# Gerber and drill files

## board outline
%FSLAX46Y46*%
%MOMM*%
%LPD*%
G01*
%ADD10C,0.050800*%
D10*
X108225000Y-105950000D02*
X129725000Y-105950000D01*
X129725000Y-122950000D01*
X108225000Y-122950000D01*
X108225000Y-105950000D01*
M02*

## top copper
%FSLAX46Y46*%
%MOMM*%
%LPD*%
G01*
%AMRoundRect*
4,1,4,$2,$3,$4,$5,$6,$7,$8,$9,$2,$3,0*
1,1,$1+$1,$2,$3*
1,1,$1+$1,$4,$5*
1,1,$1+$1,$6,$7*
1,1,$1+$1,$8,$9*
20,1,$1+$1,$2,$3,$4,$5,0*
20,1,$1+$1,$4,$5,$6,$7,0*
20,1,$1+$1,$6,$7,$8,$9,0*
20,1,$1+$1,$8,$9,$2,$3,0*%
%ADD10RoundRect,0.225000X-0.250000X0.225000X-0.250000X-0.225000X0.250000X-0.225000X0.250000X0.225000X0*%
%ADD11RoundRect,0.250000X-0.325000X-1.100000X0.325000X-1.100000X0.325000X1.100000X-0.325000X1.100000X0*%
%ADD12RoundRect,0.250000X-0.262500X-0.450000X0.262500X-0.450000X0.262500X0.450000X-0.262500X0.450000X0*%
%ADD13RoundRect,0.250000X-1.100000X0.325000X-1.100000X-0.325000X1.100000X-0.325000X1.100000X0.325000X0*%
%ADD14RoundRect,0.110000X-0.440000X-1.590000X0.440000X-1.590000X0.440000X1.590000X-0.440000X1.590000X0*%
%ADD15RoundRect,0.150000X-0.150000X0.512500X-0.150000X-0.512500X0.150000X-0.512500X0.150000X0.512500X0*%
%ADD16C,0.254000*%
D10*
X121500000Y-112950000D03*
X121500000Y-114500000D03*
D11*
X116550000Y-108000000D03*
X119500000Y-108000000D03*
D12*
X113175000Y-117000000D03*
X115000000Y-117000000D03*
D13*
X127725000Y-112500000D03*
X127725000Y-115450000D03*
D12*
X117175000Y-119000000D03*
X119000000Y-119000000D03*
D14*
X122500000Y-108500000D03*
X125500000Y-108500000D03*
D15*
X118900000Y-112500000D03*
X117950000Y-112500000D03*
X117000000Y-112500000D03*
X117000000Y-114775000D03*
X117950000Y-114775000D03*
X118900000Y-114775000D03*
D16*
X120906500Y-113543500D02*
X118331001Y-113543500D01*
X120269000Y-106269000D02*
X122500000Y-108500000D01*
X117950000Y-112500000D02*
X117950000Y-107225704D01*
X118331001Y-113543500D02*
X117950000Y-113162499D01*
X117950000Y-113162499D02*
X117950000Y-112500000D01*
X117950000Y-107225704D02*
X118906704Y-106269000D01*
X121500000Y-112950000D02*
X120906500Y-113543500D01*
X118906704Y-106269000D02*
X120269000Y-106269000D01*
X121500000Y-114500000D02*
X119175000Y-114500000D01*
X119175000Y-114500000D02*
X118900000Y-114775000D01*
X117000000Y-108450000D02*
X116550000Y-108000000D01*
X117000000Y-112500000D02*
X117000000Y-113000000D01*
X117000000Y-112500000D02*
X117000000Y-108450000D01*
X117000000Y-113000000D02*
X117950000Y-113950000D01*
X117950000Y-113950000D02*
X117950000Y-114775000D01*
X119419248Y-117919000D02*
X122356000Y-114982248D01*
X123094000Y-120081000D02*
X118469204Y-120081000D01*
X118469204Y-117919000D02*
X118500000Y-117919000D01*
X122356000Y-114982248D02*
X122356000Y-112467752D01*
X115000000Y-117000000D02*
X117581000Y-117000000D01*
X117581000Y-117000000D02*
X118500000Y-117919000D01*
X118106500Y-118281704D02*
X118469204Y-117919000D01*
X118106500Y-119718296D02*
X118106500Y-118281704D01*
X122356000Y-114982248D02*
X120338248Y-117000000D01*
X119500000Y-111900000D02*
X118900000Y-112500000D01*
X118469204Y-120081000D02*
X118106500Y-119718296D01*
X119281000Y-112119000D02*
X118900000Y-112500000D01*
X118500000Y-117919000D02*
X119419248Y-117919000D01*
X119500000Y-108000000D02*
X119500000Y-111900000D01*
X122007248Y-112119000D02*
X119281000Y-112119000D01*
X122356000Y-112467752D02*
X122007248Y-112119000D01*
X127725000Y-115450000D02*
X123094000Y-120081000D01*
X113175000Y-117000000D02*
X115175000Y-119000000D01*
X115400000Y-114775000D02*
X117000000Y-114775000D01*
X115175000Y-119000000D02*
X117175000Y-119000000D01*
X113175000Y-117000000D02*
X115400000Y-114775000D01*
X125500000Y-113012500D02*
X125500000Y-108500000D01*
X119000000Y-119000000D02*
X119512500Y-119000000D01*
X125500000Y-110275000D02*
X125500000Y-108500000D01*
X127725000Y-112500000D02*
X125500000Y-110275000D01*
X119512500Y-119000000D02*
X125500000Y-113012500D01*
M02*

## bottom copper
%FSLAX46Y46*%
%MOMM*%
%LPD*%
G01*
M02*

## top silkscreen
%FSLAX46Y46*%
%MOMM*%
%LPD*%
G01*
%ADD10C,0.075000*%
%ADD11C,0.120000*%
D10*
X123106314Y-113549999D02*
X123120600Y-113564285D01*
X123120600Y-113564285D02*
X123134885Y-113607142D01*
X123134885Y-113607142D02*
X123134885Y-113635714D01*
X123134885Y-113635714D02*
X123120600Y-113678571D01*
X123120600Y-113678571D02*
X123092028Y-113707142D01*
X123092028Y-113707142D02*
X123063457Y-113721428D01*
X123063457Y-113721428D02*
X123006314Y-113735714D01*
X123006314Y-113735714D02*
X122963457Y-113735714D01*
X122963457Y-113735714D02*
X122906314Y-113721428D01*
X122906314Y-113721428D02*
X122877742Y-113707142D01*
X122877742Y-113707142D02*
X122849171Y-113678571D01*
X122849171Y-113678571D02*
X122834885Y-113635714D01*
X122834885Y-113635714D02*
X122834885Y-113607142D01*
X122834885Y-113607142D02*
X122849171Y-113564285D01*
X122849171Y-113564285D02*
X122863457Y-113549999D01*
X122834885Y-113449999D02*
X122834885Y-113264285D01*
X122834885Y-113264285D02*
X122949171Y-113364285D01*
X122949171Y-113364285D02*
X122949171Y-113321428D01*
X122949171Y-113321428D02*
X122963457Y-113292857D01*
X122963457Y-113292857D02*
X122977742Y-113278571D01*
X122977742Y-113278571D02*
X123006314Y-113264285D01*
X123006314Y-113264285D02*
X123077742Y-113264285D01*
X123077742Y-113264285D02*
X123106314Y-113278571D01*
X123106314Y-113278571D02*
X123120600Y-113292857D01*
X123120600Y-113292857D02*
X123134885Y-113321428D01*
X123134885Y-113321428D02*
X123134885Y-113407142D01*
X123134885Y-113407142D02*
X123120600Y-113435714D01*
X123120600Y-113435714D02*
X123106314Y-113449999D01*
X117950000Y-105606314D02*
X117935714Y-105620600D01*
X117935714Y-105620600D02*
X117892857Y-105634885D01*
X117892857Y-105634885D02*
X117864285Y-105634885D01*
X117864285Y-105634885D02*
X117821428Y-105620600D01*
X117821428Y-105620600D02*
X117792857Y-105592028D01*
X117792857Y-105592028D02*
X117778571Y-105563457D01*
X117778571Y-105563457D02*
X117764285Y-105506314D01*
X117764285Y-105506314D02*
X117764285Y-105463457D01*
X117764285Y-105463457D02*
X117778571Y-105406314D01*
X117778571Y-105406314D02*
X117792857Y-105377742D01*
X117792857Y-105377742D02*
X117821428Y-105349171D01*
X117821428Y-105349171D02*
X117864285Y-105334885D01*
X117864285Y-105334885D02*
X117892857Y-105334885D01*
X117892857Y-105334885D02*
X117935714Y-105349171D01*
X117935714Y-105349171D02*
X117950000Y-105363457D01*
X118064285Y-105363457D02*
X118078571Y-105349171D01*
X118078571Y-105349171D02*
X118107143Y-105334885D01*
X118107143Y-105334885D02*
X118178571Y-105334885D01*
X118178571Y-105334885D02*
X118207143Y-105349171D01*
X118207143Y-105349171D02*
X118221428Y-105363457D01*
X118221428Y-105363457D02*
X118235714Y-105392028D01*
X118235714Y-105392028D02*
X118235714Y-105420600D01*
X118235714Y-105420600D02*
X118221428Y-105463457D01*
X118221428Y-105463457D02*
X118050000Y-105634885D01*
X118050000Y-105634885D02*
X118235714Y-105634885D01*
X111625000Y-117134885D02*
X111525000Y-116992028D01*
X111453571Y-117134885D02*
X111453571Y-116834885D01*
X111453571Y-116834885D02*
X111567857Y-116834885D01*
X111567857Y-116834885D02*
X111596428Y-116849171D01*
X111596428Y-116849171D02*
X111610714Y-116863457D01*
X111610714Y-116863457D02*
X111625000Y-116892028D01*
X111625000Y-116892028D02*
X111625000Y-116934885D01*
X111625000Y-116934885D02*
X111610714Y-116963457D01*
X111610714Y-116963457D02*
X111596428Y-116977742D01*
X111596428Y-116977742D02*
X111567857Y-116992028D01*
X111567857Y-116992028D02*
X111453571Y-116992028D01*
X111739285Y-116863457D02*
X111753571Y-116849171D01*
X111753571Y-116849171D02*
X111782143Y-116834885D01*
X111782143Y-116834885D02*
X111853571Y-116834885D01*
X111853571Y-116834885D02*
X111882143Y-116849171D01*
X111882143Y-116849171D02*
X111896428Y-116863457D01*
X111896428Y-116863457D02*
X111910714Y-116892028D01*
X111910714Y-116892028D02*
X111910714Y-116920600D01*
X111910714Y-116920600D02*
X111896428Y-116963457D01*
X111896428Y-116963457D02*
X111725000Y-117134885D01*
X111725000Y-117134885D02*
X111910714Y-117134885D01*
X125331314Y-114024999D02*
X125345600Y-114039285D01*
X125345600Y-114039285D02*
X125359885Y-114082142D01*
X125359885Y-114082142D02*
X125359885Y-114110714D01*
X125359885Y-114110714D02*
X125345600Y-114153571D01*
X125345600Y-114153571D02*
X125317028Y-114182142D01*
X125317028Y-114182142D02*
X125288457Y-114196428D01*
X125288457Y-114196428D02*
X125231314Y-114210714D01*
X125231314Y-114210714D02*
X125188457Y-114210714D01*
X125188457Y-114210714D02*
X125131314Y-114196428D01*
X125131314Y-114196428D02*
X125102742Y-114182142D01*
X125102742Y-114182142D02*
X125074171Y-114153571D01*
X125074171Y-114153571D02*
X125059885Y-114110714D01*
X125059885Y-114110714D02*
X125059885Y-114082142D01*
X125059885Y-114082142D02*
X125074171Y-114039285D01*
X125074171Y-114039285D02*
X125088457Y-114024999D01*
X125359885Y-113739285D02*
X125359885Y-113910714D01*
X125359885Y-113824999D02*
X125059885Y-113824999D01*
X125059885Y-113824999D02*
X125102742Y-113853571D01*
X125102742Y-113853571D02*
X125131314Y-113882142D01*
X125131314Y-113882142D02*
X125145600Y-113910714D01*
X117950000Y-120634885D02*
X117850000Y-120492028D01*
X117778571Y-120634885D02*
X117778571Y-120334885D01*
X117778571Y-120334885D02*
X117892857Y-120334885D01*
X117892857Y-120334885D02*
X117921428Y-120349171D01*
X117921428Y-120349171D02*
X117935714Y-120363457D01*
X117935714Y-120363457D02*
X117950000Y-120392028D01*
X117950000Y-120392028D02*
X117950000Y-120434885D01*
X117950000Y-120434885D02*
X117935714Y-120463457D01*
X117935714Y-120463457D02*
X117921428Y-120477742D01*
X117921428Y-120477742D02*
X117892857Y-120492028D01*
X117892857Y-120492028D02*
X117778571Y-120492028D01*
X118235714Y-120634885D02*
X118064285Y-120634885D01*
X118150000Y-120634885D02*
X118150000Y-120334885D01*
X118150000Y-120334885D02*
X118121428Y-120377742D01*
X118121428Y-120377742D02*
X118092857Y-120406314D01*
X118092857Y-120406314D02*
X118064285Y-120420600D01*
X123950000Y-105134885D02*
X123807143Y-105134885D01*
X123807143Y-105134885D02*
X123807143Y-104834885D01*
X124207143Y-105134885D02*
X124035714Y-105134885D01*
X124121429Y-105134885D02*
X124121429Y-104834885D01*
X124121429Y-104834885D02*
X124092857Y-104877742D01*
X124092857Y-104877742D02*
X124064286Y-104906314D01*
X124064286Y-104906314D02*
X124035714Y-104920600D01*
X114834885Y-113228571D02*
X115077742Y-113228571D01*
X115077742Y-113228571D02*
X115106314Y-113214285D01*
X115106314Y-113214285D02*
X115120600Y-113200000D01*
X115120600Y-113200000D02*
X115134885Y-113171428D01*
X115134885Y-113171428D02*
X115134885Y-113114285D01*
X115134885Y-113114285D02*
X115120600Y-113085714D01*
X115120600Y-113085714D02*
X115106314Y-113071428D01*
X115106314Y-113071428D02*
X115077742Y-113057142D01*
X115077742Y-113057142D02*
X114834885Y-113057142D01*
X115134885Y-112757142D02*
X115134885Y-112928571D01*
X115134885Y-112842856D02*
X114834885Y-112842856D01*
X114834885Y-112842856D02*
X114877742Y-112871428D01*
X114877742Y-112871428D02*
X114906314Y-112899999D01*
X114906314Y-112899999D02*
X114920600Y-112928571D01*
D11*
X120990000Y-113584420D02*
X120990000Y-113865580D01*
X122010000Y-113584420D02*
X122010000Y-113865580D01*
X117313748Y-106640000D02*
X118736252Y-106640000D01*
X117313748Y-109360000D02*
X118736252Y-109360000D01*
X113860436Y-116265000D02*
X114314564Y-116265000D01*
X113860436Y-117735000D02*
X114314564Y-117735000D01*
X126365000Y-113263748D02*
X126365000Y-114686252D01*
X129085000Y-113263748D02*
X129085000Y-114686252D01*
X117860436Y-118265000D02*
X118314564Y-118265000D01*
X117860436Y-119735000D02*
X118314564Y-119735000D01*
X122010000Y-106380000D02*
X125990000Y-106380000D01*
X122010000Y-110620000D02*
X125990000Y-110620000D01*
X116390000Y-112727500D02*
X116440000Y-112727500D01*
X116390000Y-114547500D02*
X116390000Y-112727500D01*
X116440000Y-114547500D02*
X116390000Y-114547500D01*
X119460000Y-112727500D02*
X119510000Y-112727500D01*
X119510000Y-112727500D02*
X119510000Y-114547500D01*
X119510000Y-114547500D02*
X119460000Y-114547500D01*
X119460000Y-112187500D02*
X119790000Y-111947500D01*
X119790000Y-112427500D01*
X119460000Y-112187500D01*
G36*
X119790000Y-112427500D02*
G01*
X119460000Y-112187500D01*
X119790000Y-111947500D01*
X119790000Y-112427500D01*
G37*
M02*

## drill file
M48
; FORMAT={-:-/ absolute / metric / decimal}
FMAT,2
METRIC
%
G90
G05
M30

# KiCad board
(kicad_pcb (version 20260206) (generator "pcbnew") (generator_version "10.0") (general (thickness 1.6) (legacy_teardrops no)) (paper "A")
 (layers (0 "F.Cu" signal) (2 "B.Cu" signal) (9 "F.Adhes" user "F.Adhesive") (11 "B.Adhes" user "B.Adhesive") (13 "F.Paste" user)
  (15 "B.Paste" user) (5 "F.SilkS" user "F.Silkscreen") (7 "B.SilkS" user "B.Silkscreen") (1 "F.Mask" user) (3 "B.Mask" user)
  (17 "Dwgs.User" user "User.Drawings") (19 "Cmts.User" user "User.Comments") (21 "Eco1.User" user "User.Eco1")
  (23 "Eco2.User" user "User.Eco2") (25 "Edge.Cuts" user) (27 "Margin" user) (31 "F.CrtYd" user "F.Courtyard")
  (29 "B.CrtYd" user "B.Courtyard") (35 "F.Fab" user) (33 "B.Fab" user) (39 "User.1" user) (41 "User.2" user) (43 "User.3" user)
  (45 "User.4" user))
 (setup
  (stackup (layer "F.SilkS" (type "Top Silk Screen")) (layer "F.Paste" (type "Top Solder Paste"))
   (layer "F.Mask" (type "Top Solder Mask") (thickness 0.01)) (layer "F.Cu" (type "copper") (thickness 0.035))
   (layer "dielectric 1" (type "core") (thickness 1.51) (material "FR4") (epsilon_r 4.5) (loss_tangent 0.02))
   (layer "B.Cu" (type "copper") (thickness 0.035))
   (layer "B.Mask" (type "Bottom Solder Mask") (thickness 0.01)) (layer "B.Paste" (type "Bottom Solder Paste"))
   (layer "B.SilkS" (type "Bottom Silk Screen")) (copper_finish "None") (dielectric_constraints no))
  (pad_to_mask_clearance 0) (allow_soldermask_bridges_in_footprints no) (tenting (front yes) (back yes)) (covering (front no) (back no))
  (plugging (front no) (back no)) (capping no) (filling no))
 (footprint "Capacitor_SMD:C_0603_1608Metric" (layer "F.Cu") (at 121.5 113.725 -90)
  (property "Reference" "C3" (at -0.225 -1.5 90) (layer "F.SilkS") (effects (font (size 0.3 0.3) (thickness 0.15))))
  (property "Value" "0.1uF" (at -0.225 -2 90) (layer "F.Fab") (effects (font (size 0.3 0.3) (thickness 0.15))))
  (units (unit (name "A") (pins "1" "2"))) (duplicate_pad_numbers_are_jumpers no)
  (fp_line (start -0.14058 0.51) (end 0.14058 0.51) (stroke (width 0.12) (type solid)) (layer "F.SilkS"))
  (fp_line (start -0.14058 -0.51) (end 0.14058 -0.51) (stroke (width 0.12) (type solid)) (layer "F.SilkS"))
  (pad "1" smd roundrect (at -0.775 0 270) (size 0.9 0.95) (layers "F.Cu" "F.Mask" "F.Paste") (roundrect_rratio 0.25) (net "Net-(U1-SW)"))
  (pad "2" smd roundrect (at 0.775 0 270) (size 0.9 0.95) (layers "F.Cu" "F.Mask" "F.Paste") (roundrect_rratio 0.25) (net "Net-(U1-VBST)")))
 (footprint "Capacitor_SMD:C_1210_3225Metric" (layer "F.Cu") (at 118.025 108)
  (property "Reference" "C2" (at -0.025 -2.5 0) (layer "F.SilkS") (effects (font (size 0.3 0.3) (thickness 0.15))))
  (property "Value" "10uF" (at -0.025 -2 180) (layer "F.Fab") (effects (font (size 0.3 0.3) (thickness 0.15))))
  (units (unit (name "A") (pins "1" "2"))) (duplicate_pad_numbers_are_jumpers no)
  (fp_line (start -0.711252 -1.36) (end 0.711252 -1.36) (stroke (width 0.12) (type solid)) (layer "F.SilkS"))
  (fp_line (start -0.711252 1.36) (end 0.711252 1.36) (stroke (width 0.12) (type solid)) (layer "F.SilkS"))
  (pad "1" smd roundrect (at -1.475 0) (size 1.15 2.7) (layers "F.Cu" "F.Mask" "F.Paste") (roundrect_rratio 0.217391) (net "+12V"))
  (pad "2" smd roundrect (at 1.475 0) (size 1.15 2.7) (layers "F.Cu" "F.Mask" "F.Paste") (roundrect_rratio 0.217391) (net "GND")))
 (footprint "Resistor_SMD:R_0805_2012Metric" (layer "F.Cu") (at 114.0875 117)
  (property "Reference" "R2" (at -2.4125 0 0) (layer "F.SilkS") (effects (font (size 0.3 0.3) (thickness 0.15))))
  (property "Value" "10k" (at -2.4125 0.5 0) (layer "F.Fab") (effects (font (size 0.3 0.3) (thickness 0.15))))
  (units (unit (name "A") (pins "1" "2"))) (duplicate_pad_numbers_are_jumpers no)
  (fp_line (start -0.227064 -0.735) (end 0.227064 -0.735) (stroke (width 0.12) (type solid)) (layer "F.SilkS"))
  (fp_line (start -0.227064 0.735) (end 0.227064 0.735) (stroke (width 0.12) (type solid)) (layer "F.SilkS"))
  (pad "1" smd roundrect (at -0.9125 0) (size 1.025 1.4) (layers "F.Cu" "F.Mask" "F.Paste") (roundrect_rratio 0.243902) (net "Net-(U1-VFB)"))
  (pad "2" smd roundrect (at 0.9125 0) (size 1.025 1.4) (layers "F.Cu" "F.Mask" "F.Paste") (roundrect_rratio 0.243902) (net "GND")))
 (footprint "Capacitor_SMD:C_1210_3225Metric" (layer "F.Cu") (at 127.725 113.975 -90)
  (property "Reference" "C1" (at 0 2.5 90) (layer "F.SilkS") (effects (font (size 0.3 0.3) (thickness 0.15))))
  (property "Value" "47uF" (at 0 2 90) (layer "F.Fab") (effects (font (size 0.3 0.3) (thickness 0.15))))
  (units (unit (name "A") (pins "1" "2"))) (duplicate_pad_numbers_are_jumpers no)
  (fp_line (start -0.711252 1.36) (end 0.711252 1.36) (stroke (width 0.12) (type solid)) (layer "F.SilkS"))
  (fp_line (start -0.711252 -1.36) (end 0.711252 -1.36) (stroke (width 0.12) (type solid)) (layer "F.SilkS"))
  (pad "1" smd roundrect (at -1.475 0 270) (size 1.15 2.7) (layers "F.Cu" "F.Mask" "F.Paste") (roundrect_rratio 0.217391) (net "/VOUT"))
  (pad "2" smd roundrect (at 1.475 0 270) (size 1.15 2.7) (layers "F.Cu" "F.Mask" "F.Paste") (roundrect_rratio 0.217391) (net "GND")))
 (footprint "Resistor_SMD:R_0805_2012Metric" (layer "F.Cu") (at 118.0875 119)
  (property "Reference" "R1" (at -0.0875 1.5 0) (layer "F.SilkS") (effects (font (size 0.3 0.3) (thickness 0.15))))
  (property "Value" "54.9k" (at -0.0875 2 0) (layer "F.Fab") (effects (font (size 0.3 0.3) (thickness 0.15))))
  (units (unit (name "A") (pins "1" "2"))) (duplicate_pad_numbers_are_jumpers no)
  (fp_line (start -0.227064 -0.735) (end 0.227064 -0.735) (stroke (width 0.12) (type solid)) (layer "F.SilkS"))
  (fp_line (start -0.227064 0.735) (end 0.227064 0.735) (stroke (width 0.12) (type solid)) (layer "F.SilkS"))
  (pad "1" smd roundrect (at -0.9125 0) (size 1.025 1.4) (layers "F.Cu" "F.Mask" "F.Paste") (roundrect_rratio 0.243902) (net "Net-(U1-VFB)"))
  (pad "2" smd roundrect (at 0.9125 0) (size 1.025 1.4) (layers "F.Cu" "F.Mask" "F.Paste") (roundrect_rratio 0.243902) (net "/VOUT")))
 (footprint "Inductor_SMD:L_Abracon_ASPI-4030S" (layer "F.Cu") (at 124 108.5)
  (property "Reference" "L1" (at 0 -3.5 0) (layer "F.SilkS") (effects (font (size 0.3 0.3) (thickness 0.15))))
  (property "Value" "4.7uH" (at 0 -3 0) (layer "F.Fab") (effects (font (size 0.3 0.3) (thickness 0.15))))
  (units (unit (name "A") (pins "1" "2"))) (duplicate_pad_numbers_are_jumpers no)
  (fp_line (start -1.99 -2.12) (end 1.99 -2.12) (stroke (width 0.12) (type solid)) (layer "F.SilkS"))
  (fp_line (start -1.99 2.12) (end 1.99 2.12) (stroke (width 0.12) (type solid)) (layer "F.SilkS"))
  (pad "1" smd roundrect (at -1.5 0) (size 1.1 3.4) (layers "F.Cu" "F.Mask" "F.Paste") (roundrect_rratio 0.1) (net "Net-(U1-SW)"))
  (pad "2" smd roundrect (at 1.5 0) (size 1.1 3.4) (layers "F.Cu" "F.Mask" "F.Paste") (roundrect_rratio 0.1) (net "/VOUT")))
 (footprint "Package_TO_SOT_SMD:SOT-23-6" (layer "F.Cu") (at 117.95 113.6375 -90)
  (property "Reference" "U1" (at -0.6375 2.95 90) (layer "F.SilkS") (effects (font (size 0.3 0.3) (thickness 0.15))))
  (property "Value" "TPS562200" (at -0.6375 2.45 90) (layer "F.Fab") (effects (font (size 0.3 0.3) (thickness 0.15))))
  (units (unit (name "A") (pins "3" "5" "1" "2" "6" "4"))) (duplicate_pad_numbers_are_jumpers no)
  (fp_line (start -0.91 1.56) (end -0.91 1.51) (stroke (width 0.12) (type solid)) (layer "F.SilkS"))
  (fp_line (start 0.91 1.56) (end -0.91 1.56) (stroke (width 0.12) (type solid)) (layer "F.SilkS"))
  (fp_line (start 0.91 1.51) (end 0.91 1.56) (stroke (width 0.12) (type solid)) (layer "F.SilkS"))
  (fp_line (start -0.91 -1.51) (end -0.91 -1.56) (stroke (width 0.12) (type solid)) (layer "F.SilkS"))
  (fp_line (start -0.91 -1.56) (end 0.91 -1.56) (stroke (width 0.12) (type solid)) (layer "F.SilkS"))
  (fp_line (start 0.91 -1.56) (end 0.91 -1.51) (stroke (width 0.12) (type solid)) (layer "F.SilkS"))
  (fp_poly (pts (xy -1.45 -1.51) (xy -1.69 -1.84) (xy -1.21 -1.84)) (stroke (width 0.12) (type solid)) (fill yes) (layer "F.SilkS"))
  (pad "1" smd roundrect (at -1.1375 -0.95 270) (size 1.325 0.6) (layers "F.Cu" "F.Mask" "F.Paste") (roundrect_rratio 0.25) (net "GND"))
  (pad "2" smd roundrect (at -1.1375 0 270) (size 1.325 0.6) (layers "F.Cu" "F.Mask" "F.Paste") (roundrect_rratio 0.25) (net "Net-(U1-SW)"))
  (pad "3" smd roundrect (at -1.1375 0.95 270) (size 1.325 0.6) (layers "F.Cu" "F.Mask" "F.Paste") (roundrect_rratio 0.25) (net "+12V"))
  (pad "4" smd roundrect (at 1.1375 0.95 270) (size 1.325 0.6) (layers "F.Cu" "F.Mask" "F.Paste") (roundrect_rratio 0.25)
   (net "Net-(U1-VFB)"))
  (pad "5" smd roundrect (at 1.1375 0 270) (size 1.325 0.6) (layers "F.Cu" "F.Mask" "F.Paste") (roundrect_rratio 0.25) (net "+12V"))
  (pad "6" smd roundrect (at 1.1375 -0.95 270) (size 1.325 0.6) (layers "F.Cu" "F.Mask" "F.Paste") (roundrect_rratio 0.25)
   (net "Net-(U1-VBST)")))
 (gr_rect (start 108.225 105.95) (end 129.725 122.95) (stroke (width 0.0508) (type default)) (fill no) (layer "Edge.Cuts"))
 (segment (start 120.9065 113.5435) (end 118.331001 113.5435) (width 0.254) (layer "F.Cu") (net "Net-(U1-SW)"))
 (segment (start 120.269 106.269) (end 122.5 108.5) (width 0.254) (layer "F.Cu") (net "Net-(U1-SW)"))
 (segment (start 117.95 112.5) (end 117.95 107.225704) (width 0.254) (layer "F.Cu") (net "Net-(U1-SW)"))
 (segment (start 118.331001 113.5435) (end 117.95 113.162499) (width 0.254) (layer "F.Cu") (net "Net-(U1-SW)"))
 (segment (start 117.95 113.162499) (end 117.95 112.5) (width 0.254) (layer "F.Cu") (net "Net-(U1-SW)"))
 (segment (start 117.95 107.225704) (end 118.906704 106.269) (width 0.254) (layer "F.Cu") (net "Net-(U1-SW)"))
 (segment (start 121.5 112.95) (end 120.9065 113.5435) (width 0.254) (layer "F.Cu") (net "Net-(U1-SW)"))
 (segment (start 118.906704 106.269) (end 120.269 106.269) (width 0.254) (layer "F.Cu") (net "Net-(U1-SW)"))
 (segment (start 121.5 114.5) (end 119.175 114.5) (width 0.254) (layer "F.Cu") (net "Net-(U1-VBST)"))
 (segment (start 119.175 114.5) (end 118.9 114.775) (width 0.254) (layer "F.Cu") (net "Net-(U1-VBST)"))
 (segment (start 117 108.45) (end 116.55 108) (width 0.254) (layer "F.Cu") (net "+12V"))
 (segment (start 117 112.5) (end 117 113) (width 0.254) (layer "F.Cu") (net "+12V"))
 (segment (start 117 112.5) (end 117 108.45) (width 0.254) (layer "F.Cu") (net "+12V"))
 (segment (start 117 113) (end 117.95 113.95) (width 0.254) (layer "F.Cu") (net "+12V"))
 (segment (start 117.95 113.95) (end 117.95 114.775) (width 0.254) (layer "F.Cu") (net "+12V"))
 (segment (start 119.419248 117.919) (end 122.356 114.982248) (width 0.254) (layer "F.Cu") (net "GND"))
 (segment (start 123.094 120.081) (end 118.469204 120.081) (width 0.254) (layer "F.Cu") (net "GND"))
 (segment (start 118.469204 117.919) (end 118.5 117.919) (width 0.254) (layer "F.Cu") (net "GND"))
 (segment (start 122.356 114.982248) (end 122.356 112.467752) (width 0.254) (layer "F.Cu") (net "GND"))
 (segment (start 115 117) (end 117.581 117) (width 0.254) (layer "F.Cu") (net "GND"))
 (segment (start 117.581 117) (end 118.5 117.919) (width 0.254) (layer "F.Cu") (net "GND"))
 (segment (start 118.1065 118.281704) (end 118.469204 117.919) (width 0.254) (layer "F.Cu") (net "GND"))
 (segment (start 118.1065 119.718296) (end 118.1065 118.281704) (width 0.254) (layer "F.Cu") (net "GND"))
 (segment (start 122.356 114.982248) (end 120.338248 117) (width 0.254) (layer "F.Cu") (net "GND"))
 (segment (start 119.5 111.9) (end 118.9 112.5) (width 0.254) (layer "F.Cu") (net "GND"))
 (segment (start 118.469204 120.081) (end 118.1065 119.718296) (width 0.254) (layer "F.Cu") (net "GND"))
 (segment (start 119.281 112.119) (end 118.9 112.5) (width 0.254) (layer "F.Cu") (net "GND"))
 (segment (start 118.5 117.919) (end 119.419248 117.919) (width 0.254) (layer "F.Cu") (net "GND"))
 (segment (start 119.5 108) (end 119.5 111.9) (width 0.254) (layer "F.Cu") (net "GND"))
 (segment (start 122.007248 112.119) (end 119.281 112.119) (width 0.254) (layer "F.Cu") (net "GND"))
 (segment (start 122.356 112.467752) (end 122.007248 112.119) (width 0.254) (layer "F.Cu") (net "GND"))
 (segment (start 127.725 115.45) (end 123.094 120.081) (width 0.254) (layer "F.Cu") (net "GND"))
 (segment (start 113.175 117) (end 115.175 119) (width 0.254) (layer "F.Cu") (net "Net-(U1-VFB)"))
 (segment (start 115.4 114.775) (end 117 114.775) (width 0.254) (layer "F.Cu") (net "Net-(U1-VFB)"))
 (segment (start 115.175 119) (end 117.175 119) (width 0.254) (layer "F.Cu") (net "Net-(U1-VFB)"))
 (segment (start 113.175 117) (end 115.4 114.775) (width 0.254) (layer "F.Cu") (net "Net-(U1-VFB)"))
 (segment (start 125.5 113.0125) (end 125.5 108.5) (width 0.254) (layer "F.Cu") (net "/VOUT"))
 (segment (start 119 119) (end 119.5125 119) (width 0.254) (layer "F.Cu") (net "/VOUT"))
 (segment (start 125.5 110.275) (end 125.5 108.5) (width 0.254) (layer "F.Cu") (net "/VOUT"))
 (segment (start 127.725 112.5) (end 125.5 110.275) (width 0.254) (layer "F.Cu") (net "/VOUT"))
 (segment (start 119.5125 119) (end 125.5 113.0125) (width 0.254) (layer "F.Cu") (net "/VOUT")))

